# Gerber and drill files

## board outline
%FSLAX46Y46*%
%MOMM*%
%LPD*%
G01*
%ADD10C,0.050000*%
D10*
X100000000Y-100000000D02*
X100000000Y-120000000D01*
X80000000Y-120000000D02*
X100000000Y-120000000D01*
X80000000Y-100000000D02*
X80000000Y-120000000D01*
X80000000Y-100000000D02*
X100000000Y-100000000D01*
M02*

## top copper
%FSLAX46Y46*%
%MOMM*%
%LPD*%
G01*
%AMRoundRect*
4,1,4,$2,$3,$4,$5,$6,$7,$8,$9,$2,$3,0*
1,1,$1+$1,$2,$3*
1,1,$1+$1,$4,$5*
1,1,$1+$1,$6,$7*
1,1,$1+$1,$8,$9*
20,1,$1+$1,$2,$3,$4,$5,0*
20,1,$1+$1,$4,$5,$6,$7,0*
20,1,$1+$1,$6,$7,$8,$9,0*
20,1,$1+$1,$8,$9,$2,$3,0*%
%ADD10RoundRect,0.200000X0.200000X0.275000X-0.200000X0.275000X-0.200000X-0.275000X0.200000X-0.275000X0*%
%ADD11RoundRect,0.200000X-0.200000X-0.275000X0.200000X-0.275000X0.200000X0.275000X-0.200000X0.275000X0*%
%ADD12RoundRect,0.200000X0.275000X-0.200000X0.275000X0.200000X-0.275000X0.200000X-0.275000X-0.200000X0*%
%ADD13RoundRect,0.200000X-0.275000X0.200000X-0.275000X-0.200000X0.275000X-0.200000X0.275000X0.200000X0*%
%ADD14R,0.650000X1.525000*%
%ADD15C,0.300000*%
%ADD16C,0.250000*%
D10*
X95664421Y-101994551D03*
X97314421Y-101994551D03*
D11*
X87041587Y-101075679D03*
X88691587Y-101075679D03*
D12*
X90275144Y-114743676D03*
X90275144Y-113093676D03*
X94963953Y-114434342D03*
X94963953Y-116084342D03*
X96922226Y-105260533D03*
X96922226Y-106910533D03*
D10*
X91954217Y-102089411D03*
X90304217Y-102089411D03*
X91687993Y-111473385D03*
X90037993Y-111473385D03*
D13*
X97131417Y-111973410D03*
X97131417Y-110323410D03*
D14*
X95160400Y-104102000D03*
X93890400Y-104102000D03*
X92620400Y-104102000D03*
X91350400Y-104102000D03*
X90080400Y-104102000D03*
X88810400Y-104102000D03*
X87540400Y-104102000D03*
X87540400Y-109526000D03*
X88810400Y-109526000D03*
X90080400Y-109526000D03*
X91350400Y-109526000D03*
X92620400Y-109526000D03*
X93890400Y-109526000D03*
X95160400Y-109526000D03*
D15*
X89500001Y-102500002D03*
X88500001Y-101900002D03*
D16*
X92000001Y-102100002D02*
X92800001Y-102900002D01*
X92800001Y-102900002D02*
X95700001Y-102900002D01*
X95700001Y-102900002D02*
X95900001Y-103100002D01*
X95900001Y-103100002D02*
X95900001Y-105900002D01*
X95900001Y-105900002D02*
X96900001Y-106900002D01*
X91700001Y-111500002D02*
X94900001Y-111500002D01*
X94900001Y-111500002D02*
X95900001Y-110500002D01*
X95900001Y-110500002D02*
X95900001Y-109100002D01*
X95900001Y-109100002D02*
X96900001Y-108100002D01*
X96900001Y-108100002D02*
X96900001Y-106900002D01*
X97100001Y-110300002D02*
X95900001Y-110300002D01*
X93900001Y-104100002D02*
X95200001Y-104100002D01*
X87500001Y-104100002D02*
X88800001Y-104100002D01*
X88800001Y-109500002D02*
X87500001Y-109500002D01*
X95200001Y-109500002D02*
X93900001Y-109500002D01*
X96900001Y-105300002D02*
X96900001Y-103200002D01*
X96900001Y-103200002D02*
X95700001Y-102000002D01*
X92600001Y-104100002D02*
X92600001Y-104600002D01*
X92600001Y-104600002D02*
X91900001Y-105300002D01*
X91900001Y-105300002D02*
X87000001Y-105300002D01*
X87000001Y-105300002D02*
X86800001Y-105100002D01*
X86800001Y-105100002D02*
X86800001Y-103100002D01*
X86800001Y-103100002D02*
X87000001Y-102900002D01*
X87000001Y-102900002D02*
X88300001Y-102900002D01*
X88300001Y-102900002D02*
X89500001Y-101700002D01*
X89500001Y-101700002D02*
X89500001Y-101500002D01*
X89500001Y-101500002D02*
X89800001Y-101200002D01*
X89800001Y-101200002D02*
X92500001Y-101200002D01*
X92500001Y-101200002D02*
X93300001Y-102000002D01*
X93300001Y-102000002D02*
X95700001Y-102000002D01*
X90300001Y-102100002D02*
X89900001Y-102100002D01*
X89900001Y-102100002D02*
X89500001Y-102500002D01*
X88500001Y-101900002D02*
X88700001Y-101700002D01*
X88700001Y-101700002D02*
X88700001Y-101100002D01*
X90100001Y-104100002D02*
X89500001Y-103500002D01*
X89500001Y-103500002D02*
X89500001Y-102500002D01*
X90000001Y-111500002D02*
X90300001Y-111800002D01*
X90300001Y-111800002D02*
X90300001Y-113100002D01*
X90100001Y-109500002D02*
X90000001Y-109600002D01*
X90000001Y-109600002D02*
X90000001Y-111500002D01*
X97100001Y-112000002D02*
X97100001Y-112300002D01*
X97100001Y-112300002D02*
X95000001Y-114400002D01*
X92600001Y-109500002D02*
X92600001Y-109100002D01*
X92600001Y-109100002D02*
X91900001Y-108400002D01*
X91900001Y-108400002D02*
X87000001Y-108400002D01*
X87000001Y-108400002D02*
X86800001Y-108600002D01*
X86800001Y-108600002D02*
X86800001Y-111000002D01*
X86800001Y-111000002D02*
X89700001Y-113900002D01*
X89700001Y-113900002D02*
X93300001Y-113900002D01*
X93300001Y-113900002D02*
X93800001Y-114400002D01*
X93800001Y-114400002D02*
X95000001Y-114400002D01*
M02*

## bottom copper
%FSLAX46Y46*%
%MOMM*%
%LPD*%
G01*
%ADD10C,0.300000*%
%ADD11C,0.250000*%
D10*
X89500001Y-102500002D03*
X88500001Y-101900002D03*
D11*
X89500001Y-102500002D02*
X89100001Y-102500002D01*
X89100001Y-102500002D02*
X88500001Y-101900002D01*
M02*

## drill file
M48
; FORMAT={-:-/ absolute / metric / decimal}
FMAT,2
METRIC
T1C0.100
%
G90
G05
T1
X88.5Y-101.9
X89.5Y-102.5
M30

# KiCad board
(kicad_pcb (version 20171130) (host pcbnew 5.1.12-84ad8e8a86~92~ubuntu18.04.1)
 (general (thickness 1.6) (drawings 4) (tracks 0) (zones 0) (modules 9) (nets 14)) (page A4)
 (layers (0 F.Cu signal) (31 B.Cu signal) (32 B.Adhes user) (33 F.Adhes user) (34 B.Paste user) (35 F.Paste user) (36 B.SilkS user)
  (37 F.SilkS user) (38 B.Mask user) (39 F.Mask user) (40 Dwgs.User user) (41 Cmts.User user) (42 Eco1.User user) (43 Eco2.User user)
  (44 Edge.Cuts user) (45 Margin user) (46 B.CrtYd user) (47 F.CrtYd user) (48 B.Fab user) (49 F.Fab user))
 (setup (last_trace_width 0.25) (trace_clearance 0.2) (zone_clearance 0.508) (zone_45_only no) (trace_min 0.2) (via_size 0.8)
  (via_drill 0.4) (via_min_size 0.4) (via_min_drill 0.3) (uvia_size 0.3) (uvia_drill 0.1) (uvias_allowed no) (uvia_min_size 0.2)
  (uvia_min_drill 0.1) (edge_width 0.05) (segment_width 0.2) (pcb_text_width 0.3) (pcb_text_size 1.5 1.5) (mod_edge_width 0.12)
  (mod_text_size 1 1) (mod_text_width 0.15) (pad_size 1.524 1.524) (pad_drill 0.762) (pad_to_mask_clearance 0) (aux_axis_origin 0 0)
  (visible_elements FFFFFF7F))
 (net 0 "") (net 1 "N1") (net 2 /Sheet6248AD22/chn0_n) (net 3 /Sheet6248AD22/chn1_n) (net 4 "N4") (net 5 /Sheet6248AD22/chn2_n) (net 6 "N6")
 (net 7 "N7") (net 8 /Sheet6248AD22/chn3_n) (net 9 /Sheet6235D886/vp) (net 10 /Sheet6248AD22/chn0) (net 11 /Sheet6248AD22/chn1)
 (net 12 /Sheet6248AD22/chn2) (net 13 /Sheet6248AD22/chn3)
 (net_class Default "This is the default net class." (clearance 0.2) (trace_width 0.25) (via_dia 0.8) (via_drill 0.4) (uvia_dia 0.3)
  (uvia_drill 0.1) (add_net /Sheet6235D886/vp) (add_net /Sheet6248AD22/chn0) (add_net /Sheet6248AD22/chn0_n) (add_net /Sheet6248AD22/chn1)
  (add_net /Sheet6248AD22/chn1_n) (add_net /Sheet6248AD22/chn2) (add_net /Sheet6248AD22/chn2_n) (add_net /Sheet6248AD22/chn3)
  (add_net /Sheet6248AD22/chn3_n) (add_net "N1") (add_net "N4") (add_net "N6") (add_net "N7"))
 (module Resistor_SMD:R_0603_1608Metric (layer F.Cu) (at 96.489421 101.994551 180.000000)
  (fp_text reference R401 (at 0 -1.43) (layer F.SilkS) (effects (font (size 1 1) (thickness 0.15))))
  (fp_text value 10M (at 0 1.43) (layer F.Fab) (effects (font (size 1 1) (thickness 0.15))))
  (pad 2 smd roundrect (at 0.825 0 180.000000) (size 0.8 0.95) (layers F.Cu F.Mask F.Paste) (roundrect_rratio 0.25) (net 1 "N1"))
  (pad 1 smd roundrect (at -0.825 0 180.000000) (size 0.8 0.95) (layers F.Cu F.Mask F.Paste) (roundrect_rratio 0.25)
   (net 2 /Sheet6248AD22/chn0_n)))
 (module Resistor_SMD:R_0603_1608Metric (layer F.Cu) (at 87.866587 101.075679)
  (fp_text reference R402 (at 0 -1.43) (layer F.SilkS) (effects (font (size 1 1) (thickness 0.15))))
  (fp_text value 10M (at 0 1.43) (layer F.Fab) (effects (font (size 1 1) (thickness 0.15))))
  (pad 1 smd roundrect (at -0.825 0) (size 0.8 0.95) (layers F.Cu F.Mask F.Paste) (roundrect_rratio 0.25) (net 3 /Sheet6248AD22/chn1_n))
  (pad 2 smd roundrect (at 0.825 0) (size 0.8 0.95) (layers F.Cu F.Mask F.Paste) (roundrect_rratio 0.25) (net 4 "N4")))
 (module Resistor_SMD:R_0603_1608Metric (layer F.Cu) (at 90.275144 113.918676 90.000000)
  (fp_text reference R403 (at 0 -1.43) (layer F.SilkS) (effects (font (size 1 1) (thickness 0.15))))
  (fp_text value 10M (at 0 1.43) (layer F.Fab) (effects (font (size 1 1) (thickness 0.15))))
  (pad 1 smd roundrect (at -0.825 0 90.000000) (size 0.8 0.95) (layers F.Cu F.Mask F.Paste) (roundrect_rratio 0.25)
   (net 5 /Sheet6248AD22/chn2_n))
  (pad 2 smd roundrect (at 0.825 0 90.000000) (size 0.8 0.95) (layers F.Cu F.Mask F.Paste) (roundrect_rratio 0.25) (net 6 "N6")))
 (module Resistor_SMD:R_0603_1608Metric (layer F.Cu) (at 94.963953 115.259342 90.000000)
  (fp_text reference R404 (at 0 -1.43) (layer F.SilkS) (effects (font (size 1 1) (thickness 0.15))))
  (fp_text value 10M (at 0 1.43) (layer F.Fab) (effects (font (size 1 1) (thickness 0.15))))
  (pad 2 smd roundrect (at 0.825 0 90.000000) (size 0.8 0.95) (layers F.Cu F.Mask F.Paste) (roundrect_rratio 0.25) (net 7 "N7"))
  (pad 1 smd roundrect (at -0.825 0 90.000000) (size 0.8 0.95) (layers F.Cu F.Mask F.Paste) (roundrect_rratio 0.25)
   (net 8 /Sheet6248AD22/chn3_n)))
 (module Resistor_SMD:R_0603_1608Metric (layer F.Cu) (at 96.922226 106.085533 90.000000)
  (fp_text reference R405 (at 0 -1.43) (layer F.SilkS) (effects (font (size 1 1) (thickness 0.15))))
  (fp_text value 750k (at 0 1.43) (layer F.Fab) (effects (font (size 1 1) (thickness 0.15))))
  (pad 2 smd roundrect (at 0.825 0 90.000000) (size 0.8 0.95) (layers F.Cu F.Mask F.Paste) (roundrect_rratio 0.25) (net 1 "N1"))
  (pad 1 smd roundrect (at -0.825 0 90.000000) (size 0.8 0.95) (layers F.Cu F.Mask F.Paste) (roundrect_rratio 0.25)
   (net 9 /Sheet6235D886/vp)))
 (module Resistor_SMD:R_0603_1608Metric (layer F.Cu) (at 91.129217 102.089411 180.000000)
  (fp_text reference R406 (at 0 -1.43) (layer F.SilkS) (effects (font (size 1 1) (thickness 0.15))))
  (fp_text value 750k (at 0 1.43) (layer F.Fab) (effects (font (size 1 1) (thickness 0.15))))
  (pad 1 smd roundrect (at -0.825 0 180.000000) (size 0.8 0.95) (layers F.Cu F.Mask F.Paste) (roundrect_rratio 0.25)
   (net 9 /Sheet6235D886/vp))
  (pad 2 smd roundrect (at 0.825 0 180.000000) (size 0.8 0.95) (layers F.Cu F.Mask F.Paste) (roundrect_rratio 0.25) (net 4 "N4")))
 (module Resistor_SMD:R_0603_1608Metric (layer F.Cu) (at 90.862993 111.473385 180.000000)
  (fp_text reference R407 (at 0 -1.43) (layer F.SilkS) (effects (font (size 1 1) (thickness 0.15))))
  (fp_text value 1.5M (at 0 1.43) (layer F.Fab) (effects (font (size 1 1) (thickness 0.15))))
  (pad 1 smd roundrect (at -0.825 0 180.000000) (size 0.8 0.95) (layers F.Cu F.Mask F.Paste) (roundrect_rratio 0.25)
   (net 9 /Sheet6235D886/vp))
  (pad 2 smd roundrect (at 0.825 0 180.000000) (size 0.8 0.95) (layers F.Cu F.Mask F.Paste) (roundrect_rratio 0.25) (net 6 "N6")))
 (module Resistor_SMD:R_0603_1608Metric (layer F.Cu) (at 97.131417 111.148410 270.000000)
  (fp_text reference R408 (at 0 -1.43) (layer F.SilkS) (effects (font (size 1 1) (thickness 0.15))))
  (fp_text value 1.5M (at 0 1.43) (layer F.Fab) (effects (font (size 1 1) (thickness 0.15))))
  (pad 2 smd roundrect (at 0.825 0 270.000000) (size 0.8 0.95) (layers F.Cu F.Mask F.Paste) (roundrect_rratio 0.25) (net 7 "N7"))
  (pad 1 smd roundrect (at -0.825 0 270.000000) (size 0.8 0.95) (layers F.Cu F.Mask F.Paste) (roundrect_rratio 0.25)
   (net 9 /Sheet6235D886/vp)))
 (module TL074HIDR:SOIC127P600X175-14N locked (layer F.Cu) (at 91.350400 106.814000 270.000000)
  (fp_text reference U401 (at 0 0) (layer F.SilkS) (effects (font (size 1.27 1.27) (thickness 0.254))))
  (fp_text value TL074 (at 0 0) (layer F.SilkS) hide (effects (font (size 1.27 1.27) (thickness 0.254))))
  (pad 1 smd rect (at -2.712 -3.81) (size 0.65 1.525) (layers F.Cu F.Mask F.Paste) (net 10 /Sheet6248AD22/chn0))
  (pad 2 smd rect (at -2.712 -2.54) (size 0.65 1.525) (layers F.Cu F.Mask F.Paste) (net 10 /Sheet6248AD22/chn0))
  (pad 3 smd rect (at -2.712 -1.27) (size 0.65 1.525) (layers F.Cu F.Mask F.Paste) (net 1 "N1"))
  (pad 4 smd rect (at -2.712 0) (size 0.65 1.525) (layers F.Cu F.Mask F.Paste))
  (pad 5 smd rect (at -2.712 1.27) (size 0.65 1.525) (layers F.Cu F.Mask F.Paste) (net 4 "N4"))
  (pad 6 smd rect (at -2.712 2.54) (size 0.65 1.525) (layers F.Cu F.Mask F.Paste) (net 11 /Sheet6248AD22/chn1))
  (pad 7 smd rect (at -2.712 3.81) (size 0.65 1.525) (layers F.Cu F.Mask F.Paste) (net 11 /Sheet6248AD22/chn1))
  (pad 8 smd rect (at 2.712 3.81) (size 0.65 1.525) (layers F.Cu F.Mask F.Paste) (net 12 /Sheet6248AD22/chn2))
  (pad 9 smd rect (at 2.712 2.54) (size 0.65 1.525) (layers F.Cu F.Mask F.Paste) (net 12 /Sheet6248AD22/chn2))
  (pad 10 smd rect (at 2.712 1.27) (size 0.65 1.525) (layers F.Cu F.Mask F.Paste) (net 6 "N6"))
  (pad 11 smd rect (at 2.712 0) (size 0.65 1.525) (layers F.Cu F.Mask F.Paste))
  (pad 12 smd rect (at 2.712 -1.27) (size 0.65 1.525) (layers F.Cu F.Mask F.Paste) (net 7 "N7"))
  (pad 13 smd rect (at 2.712 -2.54) (size 0.65 1.525) (layers F.Cu F.Mask F.Paste) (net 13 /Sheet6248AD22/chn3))
  (pad 14 smd rect (at 2.712 -3.81) (size 0.65 1.525) (layers F.Cu F.Mask F.Paste) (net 13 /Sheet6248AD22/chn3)))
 (gr_line (start 100 100) (end 100 120) (layer Edge.Cuts) (width 0.05))
 (gr_line (start 80 120) (end 100 120) (layer Edge.Cuts) (width 0.05))
 (gr_line (start 80 100) (end 80 120) (layer Edge.Cuts) (width 0.05))
 (gr_line (start 80 100) (end 100 100) (layer Edge.Cuts) (width 0.05))
 (segment (start 92.000001 102.100002) (end 92.800001 102.900002) (width 0.250000) (layer F.Cu) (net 9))
 (segment (start 92.800001 102.900002) (end 95.700001 102.900002) (width 0.250000) (layer F.Cu) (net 9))
 (segment (start 95.700001 102.900002) (end 95.900001 103.100002) (width 0.250000) (layer F.Cu) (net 9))
 (segment (start 95.900001 103.100002) (end 95.900001 105.900002) (width 0.250000) (layer F.Cu) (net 9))
 (segment (start 95.900001 105.900002) (end 96.900001 106.900002) (width 0.250000) (layer F.Cu) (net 9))
 (segment (start 91.700001 111.500002) (end 94.900001 111.500002) (width 0.250000) (layer F.Cu) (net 9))
 (segment (start 94.900001 111.500002) (end 95.900001 110.500002) (width 0.250000) (layer F.Cu) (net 9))
 (segment (start 95.900001 110.500002) (end 95.900001 109.100002) (width 0.250000) (layer F.Cu) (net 9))
 (segment (start 95.900001 109.100002) (end 96.900001 108.100002) (width 0.250000) (layer F.Cu) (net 9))
 (segment (start 96.900001 108.100002) (end 96.900001 106.900002) (width 0.250000) (layer F.Cu) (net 9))
 (segment (start 97.100001 110.300002) (end 95.900001 110.300002) (width 0.250000) (layer F.Cu) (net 9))
 (segment (start 93.900001 104.100002) (end 95.200001 104.100002) (width 0.250000) (layer F.Cu) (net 10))
 (segment (start 87.500001 104.100002) (end 88.800001 104.100002) (width 0.250000) (layer F.Cu) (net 11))
 (segment (start 88.800001 109.500002) (end 87.500001 109.500002) (width 0.250000) (layer F.Cu) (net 12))
 (segment (start 95.200001 109.500002) (end 93.900001 109.500002) (width 0.250000) (layer F.Cu) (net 13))
 (segment (start 96.900001 105.300002) (end 96.900001 103.200002) (width 0.250000) (layer F.Cu) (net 1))
 (segment (start 96.900001 103.200002) (end 95.700001 102.000002) (width 0.250000) (layer F.Cu) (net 1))
 (segment (start 92.600001 104.100002) (end 92.600001 104.600002) (width 0.250000) (layer F.Cu) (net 1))
 (segment (start 92.600001 104.600002) (end 91.900001 105.300002) (width 0.250000) (layer F.Cu) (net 1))
 (segment (start 91.900001 105.300002) (end 87.000001 105.300002) (width 0.250000) (layer F.Cu) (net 1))
 (segment (start 87.000001 105.300002) (end 86.800001 105.100002) (width 0.250000) (layer F.Cu) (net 1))
 (segment (start 86.800001 105.100002) (end 86.800001 103.100002) (width 0.250000) (layer F.Cu) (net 1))
 (segment (start 86.800001 103.100002) (end 87.000001 102.900002) (width 0.250000) (layer F.Cu) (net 1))
 (segment (start 87.000001 102.900002) (end 88.300001 102.900002) (width 0.250000) (layer F.Cu) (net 1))
 (segment (start 88.300001 102.900002) (end 89.500001 101.700002) (width 0.250000) (layer F.Cu) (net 1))
 (segment (start 89.500001 101.700002) (end 89.500001 101.500002) (width 0.250000) (layer F.Cu) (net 1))
 (segment (start 89.500001 101.500002) (end 89.800001 101.200002) (width 0.250000) (layer F.Cu) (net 1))
 (segment (start 89.800001 101.200002) (end 92.500001 101.200002) (width 0.250000) (layer F.Cu) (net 1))
 (segment (start 92.500001 101.200002) (end 93.300001 102.000002) (width 0.250000) (layer F.Cu) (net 1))
 (segment (start 93.300001 102.000002) (end 95.700001 102.000002) (width 0.250000) (layer F.Cu) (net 1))
 (segment (start 90.300001 102.100002) (end 89.900001 102.100002) (width 0.250000) (layer F.Cu) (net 4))
 (segment (start 89.900001 102.100002) (end 89.500001 102.500002) (width 0.250000) (layer F.Cu) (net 4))
 (segment (start 89.500001 102.500002) (end 89.100001 102.500002) (width 0.250000) (layer B.Cu) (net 4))
 (segment (start 89.100001 102.500002) (end 88.500001 101.900002) (width 0.250000) (layer B.Cu) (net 4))
 (segment (start 88.500001 101.900002) (end 88.700001 101.700002) (width 0.250000) (layer F.Cu) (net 4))
 (segment (start 88.700001 101.700002) (end 88.700001 101.100002) (width 0.250000) (layer F.Cu) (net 4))
 (segment (start 90.100001 104.100002) (end 89.500001 103.500002) (width 0.250000) (layer F.Cu) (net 4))
 (segment (start 89.500001 103.500002) (end 89.500001 102.500002) (width 0.250000) (layer F.Cu) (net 4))
 (via micro (at 89.500001 102.500002) (size 0.300000) (drill 0.100000) (layers F.Cu B.Cu) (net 4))
 (via micro (at 88.500001 101.900002) (size 0.300000) (drill 0.100000) (layers F.Cu B.Cu) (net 4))
 (segment (start 90.000001 111.500002) (end 90.300001 111.800002) (width 0.250000) (layer F.Cu) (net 6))
 (segment (start 90.300001 111.800002) (end 90.300001 113.100002) (width 0.250000) (layer F.Cu) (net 6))
 (segment (start 90.100001 109.500002) (end 90.000001 109.600002) (width 0.250000) (layer F.Cu) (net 6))
 (segment (start 90.000001 109.600002) (end 90.000001 111.500002) (width 0.250000) (layer F.Cu) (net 6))
 (segment (start 97.100001 112.000002) (end 97.100001 112.300002) (width 0.250000) (layer F.Cu) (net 7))
 (segment (start 97.100001 112.300002) (end 95.000001 114.400002) (width 0.250000) (layer F.Cu) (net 7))
 (segment (start 92.600001 109.500002) (end 92.600001 109.100002) (width 0.250000) (layer F.Cu) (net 7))
 (segment (start 92.600001 109.100002) (end 91.900001 108.400002) (width 0.250000) (layer F.Cu) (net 7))
 (segment (start 91.900001 108.400002) (end 87.000001 108.400002) (width 0.250000) (layer F.Cu) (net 7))
 (segment (start 87.000001 108.400002) (end 86.800001 108.600002) (width 0.250000) (layer F.Cu) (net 7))
 (segment (start 86.800001 108.600002) (end 86.800001 111.000002) (width 0.250000) (layer F.Cu) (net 7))
 (segment (start 86.800001 111.000002) (end 89.700001 113.900002) (width 0.250000) (layer F.Cu) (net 7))
 (segment (start 89.700001 113.900002) (end 93.300001 113.900002) (width 0.250000) (layer F.Cu) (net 7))
 (segment (start 93.300001 113.900002) (end 93.800001 114.400002) (width 0.250000) (layer F.Cu) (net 7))
 (segment (start 93.800001 114.400002) (end 95.000001 114.400002) (width 0.250000) (layer F.Cu) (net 7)))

